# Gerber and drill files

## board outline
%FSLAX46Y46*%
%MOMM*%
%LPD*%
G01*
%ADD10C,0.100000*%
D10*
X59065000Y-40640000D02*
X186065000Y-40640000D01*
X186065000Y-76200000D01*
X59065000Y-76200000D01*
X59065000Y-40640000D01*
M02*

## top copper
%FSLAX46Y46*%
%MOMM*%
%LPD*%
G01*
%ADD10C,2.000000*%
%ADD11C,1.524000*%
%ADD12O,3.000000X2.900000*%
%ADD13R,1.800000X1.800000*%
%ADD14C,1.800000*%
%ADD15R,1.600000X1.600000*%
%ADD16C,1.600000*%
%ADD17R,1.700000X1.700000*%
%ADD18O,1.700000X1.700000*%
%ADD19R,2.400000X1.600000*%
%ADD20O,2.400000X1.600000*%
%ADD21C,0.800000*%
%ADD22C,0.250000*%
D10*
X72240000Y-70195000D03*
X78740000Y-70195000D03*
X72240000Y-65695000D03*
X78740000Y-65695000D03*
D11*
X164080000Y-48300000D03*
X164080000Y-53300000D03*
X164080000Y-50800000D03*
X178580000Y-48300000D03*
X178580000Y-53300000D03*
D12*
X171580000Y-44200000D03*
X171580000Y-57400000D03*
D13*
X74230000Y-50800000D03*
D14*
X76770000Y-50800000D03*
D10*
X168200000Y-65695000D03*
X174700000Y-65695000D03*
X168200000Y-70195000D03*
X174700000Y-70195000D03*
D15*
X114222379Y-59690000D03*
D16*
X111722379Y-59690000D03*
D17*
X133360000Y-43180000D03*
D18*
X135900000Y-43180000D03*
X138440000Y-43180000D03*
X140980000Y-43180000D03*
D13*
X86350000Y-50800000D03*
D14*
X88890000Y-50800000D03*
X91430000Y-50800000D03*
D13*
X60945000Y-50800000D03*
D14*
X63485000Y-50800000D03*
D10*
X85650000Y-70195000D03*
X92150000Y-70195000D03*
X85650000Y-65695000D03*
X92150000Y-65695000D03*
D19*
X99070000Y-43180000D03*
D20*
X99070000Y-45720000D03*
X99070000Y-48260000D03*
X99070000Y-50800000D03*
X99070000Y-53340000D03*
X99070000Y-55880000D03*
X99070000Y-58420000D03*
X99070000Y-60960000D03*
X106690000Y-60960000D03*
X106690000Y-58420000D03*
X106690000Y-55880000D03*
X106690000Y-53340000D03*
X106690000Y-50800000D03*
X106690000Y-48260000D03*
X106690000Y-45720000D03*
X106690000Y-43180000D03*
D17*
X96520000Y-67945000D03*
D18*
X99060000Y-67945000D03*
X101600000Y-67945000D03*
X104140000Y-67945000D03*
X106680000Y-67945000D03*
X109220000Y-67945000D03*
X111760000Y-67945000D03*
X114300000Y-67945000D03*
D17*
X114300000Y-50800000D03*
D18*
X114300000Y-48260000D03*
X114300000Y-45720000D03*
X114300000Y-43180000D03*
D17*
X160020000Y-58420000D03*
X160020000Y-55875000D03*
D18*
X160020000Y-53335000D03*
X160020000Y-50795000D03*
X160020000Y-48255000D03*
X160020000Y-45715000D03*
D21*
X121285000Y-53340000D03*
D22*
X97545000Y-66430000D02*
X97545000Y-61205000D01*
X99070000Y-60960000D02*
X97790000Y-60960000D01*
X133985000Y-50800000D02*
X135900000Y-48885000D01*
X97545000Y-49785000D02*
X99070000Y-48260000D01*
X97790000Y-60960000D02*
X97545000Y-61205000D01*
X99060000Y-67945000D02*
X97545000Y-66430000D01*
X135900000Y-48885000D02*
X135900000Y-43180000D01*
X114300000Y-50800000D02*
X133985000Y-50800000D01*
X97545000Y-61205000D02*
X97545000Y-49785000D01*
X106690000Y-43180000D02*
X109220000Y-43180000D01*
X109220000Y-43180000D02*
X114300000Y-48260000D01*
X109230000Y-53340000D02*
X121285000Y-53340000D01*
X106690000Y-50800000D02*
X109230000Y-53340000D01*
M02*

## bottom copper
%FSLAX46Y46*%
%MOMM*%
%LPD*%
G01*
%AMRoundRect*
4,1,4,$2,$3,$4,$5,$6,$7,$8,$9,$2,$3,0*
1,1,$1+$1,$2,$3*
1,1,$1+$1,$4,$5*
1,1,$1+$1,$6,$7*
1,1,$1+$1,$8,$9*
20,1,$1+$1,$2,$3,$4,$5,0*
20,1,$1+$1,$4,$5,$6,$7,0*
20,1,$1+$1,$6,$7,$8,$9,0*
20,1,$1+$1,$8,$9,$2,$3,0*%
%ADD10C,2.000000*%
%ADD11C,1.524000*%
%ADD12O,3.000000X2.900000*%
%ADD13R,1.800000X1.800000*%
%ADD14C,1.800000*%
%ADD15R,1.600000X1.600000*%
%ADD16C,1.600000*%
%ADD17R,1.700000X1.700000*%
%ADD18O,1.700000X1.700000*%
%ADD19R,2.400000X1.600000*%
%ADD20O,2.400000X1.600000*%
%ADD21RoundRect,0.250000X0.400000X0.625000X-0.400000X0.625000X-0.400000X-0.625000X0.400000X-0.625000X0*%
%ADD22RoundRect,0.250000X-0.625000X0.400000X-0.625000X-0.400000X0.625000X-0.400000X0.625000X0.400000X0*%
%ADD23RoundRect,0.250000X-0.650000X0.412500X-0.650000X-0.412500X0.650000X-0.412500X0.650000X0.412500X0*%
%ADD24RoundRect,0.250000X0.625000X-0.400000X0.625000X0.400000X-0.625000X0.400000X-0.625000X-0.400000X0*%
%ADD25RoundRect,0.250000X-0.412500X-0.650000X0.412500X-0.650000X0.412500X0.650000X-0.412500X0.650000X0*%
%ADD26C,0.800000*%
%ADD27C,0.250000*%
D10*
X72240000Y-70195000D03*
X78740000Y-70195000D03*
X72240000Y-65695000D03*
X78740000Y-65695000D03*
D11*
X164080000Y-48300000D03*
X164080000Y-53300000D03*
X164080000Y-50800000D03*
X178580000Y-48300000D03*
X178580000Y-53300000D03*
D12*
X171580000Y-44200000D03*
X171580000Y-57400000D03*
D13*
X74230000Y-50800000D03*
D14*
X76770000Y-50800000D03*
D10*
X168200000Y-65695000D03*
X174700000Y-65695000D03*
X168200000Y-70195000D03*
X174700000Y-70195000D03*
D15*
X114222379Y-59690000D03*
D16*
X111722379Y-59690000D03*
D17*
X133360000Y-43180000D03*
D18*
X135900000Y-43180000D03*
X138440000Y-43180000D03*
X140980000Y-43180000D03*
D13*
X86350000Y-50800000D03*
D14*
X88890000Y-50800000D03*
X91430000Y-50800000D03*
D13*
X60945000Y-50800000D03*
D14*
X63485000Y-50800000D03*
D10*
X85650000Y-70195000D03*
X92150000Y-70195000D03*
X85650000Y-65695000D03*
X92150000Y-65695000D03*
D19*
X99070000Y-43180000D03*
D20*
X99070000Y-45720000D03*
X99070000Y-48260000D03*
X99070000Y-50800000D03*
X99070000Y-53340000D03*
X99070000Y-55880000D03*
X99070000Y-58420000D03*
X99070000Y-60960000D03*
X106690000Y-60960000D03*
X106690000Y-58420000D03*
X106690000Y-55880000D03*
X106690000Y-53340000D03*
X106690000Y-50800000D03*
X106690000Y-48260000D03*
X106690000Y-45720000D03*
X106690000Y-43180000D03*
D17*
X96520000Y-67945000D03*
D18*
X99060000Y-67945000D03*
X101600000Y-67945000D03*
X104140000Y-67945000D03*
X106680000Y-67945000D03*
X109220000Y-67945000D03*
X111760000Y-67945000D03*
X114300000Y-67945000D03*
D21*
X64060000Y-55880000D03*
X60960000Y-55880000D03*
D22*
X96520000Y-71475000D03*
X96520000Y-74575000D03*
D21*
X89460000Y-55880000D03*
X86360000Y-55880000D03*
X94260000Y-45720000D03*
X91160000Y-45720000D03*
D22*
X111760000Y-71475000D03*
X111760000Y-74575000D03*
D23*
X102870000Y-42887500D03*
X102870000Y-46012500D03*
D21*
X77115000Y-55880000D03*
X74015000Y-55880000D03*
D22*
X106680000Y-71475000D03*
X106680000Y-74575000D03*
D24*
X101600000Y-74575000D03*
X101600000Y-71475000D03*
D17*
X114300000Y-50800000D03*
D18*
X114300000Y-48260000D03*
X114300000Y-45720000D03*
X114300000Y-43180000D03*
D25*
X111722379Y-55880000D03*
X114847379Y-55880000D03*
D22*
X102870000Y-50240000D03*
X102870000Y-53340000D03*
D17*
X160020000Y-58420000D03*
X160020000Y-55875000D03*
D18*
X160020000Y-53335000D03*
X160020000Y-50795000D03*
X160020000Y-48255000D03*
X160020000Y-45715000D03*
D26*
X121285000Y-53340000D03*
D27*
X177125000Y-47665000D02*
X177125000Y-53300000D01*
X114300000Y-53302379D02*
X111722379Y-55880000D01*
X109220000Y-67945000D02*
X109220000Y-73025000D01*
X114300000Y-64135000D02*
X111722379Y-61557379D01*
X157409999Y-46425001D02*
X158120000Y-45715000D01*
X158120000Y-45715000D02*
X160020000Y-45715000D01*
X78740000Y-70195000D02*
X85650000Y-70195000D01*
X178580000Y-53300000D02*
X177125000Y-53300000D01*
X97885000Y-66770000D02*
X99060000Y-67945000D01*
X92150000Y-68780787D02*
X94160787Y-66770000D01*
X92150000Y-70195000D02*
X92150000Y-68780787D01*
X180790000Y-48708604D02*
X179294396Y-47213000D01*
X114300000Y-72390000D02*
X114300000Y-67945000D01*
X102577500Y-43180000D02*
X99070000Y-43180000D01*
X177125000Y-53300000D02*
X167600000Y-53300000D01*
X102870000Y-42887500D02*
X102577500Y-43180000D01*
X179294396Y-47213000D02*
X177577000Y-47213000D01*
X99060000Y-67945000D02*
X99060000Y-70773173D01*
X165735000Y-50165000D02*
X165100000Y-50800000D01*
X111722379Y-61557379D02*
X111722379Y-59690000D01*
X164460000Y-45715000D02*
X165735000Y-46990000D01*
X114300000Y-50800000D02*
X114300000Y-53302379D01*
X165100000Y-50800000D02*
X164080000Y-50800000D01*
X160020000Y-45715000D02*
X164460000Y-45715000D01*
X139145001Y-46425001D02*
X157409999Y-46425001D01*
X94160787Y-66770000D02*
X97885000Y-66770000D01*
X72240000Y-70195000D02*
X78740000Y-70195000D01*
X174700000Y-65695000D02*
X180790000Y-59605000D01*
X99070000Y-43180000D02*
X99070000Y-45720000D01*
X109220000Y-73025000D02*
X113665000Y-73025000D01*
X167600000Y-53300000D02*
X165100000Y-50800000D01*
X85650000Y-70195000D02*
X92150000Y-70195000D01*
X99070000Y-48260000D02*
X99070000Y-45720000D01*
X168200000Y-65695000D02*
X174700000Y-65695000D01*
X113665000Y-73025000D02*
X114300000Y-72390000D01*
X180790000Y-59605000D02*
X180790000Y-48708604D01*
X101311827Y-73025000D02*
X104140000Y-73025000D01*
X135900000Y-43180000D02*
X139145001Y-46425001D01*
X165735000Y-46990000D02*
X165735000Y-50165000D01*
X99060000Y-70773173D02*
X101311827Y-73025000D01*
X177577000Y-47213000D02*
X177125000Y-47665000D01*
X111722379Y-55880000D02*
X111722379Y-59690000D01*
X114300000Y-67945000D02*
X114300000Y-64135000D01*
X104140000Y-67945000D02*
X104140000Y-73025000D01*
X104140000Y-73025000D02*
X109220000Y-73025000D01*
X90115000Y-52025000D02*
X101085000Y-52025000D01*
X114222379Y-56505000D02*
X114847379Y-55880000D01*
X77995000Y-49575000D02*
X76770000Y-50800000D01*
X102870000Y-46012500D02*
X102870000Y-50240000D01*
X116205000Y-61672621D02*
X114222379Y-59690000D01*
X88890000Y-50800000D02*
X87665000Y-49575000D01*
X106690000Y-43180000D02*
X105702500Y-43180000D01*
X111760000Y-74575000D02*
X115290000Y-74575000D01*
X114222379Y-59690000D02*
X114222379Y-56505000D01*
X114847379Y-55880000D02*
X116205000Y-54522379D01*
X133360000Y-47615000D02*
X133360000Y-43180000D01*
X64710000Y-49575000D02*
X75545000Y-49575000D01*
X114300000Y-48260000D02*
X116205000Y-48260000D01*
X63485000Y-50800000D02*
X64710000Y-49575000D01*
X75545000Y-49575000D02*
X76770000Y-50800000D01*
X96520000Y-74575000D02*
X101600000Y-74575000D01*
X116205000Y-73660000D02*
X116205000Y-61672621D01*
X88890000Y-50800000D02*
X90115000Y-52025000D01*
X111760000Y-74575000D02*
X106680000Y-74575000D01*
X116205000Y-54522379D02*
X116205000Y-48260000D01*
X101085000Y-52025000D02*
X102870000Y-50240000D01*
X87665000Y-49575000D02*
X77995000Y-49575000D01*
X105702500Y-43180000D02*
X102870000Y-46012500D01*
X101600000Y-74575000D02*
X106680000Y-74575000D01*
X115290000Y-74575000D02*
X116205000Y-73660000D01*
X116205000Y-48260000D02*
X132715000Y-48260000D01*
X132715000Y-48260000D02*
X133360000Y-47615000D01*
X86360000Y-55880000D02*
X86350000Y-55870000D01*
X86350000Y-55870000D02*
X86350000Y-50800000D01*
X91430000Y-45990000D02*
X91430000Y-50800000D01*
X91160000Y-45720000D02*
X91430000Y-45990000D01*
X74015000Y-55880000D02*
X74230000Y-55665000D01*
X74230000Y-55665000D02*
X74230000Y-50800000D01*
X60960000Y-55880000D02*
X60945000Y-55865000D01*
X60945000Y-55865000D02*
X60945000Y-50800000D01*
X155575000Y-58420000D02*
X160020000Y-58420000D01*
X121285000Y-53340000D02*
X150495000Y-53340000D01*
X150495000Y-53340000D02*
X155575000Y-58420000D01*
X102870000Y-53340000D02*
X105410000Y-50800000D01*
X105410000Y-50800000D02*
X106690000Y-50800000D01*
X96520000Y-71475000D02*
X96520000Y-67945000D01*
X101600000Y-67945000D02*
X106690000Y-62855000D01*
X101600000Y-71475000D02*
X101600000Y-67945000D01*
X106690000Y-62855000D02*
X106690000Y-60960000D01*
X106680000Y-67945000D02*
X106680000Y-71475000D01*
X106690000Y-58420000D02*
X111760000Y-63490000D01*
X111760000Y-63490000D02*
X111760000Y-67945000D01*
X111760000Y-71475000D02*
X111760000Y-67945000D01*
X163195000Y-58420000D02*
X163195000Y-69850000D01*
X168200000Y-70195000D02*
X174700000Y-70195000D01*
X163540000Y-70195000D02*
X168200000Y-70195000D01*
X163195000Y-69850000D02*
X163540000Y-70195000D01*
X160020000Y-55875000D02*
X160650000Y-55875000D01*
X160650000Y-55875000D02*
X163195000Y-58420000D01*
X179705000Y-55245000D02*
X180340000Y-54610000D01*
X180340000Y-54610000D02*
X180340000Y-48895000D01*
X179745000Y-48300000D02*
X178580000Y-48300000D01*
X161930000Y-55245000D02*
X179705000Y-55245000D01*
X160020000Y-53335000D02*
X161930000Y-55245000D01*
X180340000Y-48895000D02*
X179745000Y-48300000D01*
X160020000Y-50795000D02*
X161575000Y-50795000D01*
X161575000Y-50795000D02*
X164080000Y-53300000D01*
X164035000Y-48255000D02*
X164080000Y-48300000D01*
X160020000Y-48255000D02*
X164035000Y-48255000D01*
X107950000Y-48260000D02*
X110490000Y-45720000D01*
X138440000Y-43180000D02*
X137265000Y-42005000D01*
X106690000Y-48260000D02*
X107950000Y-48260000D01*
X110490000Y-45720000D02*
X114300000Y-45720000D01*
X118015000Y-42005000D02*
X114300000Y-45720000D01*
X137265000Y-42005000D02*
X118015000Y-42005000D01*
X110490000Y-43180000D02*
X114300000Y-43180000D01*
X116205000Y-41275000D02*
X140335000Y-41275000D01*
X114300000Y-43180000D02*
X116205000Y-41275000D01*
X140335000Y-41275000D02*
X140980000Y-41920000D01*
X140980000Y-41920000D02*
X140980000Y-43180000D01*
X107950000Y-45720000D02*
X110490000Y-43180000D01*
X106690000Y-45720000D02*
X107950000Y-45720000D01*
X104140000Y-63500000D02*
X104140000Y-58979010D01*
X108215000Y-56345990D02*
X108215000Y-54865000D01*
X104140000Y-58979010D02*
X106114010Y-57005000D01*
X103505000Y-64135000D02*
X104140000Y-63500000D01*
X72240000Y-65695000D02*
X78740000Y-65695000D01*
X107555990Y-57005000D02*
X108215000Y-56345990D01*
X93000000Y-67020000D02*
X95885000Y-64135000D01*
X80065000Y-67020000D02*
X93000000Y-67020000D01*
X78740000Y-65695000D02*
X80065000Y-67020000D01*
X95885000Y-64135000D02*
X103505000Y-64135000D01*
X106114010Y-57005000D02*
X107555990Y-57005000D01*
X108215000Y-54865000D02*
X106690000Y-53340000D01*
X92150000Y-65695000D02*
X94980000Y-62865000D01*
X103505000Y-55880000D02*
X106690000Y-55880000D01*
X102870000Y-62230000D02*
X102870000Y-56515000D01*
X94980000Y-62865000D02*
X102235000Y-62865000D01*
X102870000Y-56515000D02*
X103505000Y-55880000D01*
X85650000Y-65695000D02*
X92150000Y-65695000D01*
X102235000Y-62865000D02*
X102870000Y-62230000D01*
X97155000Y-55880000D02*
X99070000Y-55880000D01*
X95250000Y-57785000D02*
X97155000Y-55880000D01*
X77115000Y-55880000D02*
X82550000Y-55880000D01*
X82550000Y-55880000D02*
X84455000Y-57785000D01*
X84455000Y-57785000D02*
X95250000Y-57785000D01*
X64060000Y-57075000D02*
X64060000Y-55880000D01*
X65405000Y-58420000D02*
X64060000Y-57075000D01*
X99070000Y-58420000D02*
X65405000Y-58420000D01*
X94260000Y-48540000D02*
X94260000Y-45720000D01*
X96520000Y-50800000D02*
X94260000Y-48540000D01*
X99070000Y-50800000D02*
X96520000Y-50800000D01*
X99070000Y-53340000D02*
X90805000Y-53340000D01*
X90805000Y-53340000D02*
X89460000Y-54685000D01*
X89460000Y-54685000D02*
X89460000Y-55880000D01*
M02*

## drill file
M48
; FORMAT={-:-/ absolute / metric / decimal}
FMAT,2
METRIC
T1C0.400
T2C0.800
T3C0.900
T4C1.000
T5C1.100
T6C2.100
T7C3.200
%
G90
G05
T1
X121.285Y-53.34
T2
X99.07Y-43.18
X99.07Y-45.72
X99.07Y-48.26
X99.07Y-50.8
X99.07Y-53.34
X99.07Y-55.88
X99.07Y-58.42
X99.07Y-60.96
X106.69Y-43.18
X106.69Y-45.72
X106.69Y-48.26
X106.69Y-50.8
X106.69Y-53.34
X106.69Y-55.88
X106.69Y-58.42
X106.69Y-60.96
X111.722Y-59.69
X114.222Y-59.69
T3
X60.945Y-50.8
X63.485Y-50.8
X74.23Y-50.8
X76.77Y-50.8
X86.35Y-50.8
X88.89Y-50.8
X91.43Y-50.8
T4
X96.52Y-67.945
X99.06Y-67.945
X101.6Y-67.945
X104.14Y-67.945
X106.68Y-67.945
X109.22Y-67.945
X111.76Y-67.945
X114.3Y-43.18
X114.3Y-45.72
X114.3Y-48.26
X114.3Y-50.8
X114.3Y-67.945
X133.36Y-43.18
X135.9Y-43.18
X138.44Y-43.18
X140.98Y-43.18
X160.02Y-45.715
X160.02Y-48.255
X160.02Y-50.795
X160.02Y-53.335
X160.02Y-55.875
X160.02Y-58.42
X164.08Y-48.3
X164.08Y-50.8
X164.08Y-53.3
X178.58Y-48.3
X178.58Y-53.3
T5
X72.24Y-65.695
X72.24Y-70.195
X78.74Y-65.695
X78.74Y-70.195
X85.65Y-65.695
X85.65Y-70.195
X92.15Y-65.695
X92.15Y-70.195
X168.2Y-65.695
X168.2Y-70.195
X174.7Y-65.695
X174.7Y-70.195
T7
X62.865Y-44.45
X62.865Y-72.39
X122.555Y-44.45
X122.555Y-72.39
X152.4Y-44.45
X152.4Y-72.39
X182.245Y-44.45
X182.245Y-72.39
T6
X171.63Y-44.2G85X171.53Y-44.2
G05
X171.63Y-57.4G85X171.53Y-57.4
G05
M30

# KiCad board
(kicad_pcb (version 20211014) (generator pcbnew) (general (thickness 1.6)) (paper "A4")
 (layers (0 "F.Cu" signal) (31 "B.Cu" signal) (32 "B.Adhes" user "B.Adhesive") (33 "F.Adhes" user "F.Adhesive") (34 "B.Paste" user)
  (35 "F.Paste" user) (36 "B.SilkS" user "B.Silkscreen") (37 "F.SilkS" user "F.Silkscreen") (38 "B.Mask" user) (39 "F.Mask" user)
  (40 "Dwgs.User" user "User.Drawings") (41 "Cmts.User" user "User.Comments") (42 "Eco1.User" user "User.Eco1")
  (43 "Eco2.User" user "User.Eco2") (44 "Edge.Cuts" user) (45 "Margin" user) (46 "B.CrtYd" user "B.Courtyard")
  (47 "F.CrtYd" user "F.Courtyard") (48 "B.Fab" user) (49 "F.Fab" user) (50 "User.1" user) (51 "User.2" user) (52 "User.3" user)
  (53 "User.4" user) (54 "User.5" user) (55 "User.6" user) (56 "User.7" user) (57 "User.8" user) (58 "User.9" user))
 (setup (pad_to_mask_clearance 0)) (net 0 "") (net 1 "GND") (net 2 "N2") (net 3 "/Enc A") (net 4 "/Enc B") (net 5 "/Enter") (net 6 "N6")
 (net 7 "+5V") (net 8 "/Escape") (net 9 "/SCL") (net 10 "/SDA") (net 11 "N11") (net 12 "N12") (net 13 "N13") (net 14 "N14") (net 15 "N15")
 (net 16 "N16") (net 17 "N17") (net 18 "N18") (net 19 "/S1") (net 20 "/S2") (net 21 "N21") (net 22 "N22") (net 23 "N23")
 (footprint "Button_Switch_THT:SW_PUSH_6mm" (layer "F.Cu") (at 78.74 70.195 180)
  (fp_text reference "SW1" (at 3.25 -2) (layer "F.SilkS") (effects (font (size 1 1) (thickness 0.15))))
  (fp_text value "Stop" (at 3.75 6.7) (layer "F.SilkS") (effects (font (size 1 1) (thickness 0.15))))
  (pad "1" thru_hole circle (at 6.5 0 270) (size 2 2) (drill 1.1) (layers *.Cu *.Mask) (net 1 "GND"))
  (pad "1" thru_hole circle (at 0 0 270) (size 2 2) (drill 1.1) (layers *.Cu *.Mask) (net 1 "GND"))
  (pad "2" thru_hole circle (at 6.5 4.5 270) (size 2 2) (drill 1.1) (layers *.Cu *.Mask) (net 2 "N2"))
  (pad "2" thru_hole circle (at 0 4.5 270) (size 2 2) (drill 1.1) (layers *.Cu *.Mask) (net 2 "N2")))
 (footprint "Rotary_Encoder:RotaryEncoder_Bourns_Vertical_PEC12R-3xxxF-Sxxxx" (layer "F.Cu") (at 164.08 48.3)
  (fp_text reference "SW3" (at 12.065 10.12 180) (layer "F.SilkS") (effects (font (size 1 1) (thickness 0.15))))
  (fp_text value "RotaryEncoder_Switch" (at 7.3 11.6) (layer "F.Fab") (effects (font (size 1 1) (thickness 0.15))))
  (pad "A" thru_hole circle (at 0 0 270) (size 1.524 1.524) (drill 1) (layers *.Cu *.Mask) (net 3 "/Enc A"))
  (pad "B" thru_hole circle (at 0 5 270) (size 1.524 1.524) (drill 1) (layers *.Cu *.Mask) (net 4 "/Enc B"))
  (pad "C" thru_hole circle (at 0 2.5 270) (size 1.524 1.524) (drill 1) (layers *.Cu *.Mask) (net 1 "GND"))
  (pad "S1" thru_hole circle (at 14.5 0 270) (size 1.524 1.524) (drill 1) (layers *.Cu *.Mask) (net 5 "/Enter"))
  (pad "S2" thru_hole circle (at 14.5 5 270) (size 1.524 1.524) (drill 1) (layers *.Cu *.Mask) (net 1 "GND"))
  (pad "SH" thru_hole oval (at 7.5 -4.1 270) (size 2.9 3) (drill oval 2.1 2.2) (layers *.Cu *.Mask))
  (pad "SH" thru_hole oval (at 7.5 9.1 270) (size 2.9 3) (drill oval 2.1 2.2) (layers *.Cu *.Mask)))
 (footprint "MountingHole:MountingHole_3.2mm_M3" (layer "F.Cu") (at 62.865 72.39)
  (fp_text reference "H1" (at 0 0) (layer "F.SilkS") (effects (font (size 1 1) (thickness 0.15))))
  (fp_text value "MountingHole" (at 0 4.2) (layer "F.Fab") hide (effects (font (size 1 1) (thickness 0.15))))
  (pad "" np_thru_hole circle (at 0 0) (size 3.2 3.2) (drill 3.2) (layers *.Cu *.Mask)))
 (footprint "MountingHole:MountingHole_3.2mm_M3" (layer "F.Cu") (at 122.555 44.45)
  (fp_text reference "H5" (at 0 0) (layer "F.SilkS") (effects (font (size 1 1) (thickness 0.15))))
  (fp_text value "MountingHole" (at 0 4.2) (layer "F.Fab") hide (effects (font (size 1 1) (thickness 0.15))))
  (pad "" np_thru_hole circle (at 0 0) (size 3.2 3.2) (drill 3.2) (layers *.Cu *.Mask)))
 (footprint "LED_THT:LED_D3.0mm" (layer "F.Cu") (at 74.23 50.8)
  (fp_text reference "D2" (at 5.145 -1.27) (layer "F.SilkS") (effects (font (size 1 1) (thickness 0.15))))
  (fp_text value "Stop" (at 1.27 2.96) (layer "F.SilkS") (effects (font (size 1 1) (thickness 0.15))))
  (pad "1" thru_hole rect (at 0 0) (size 1.8 1.8) (drill 0.9) (layers *.Cu *.Mask) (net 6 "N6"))
  (pad "2" thru_hole circle (at 2.54 0) (size 1.8 1.8) (drill 0.9) (layers *.Cu *.Mask) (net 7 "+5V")))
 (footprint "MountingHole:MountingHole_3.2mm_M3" (layer "F.Cu") (at 182.245 72.39)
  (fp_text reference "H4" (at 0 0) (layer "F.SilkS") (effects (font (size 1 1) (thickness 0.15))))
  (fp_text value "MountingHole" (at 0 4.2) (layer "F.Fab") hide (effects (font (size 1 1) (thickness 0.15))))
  (pad "" np_thru_hole circle (at 0 0) (size 3.2 3.2) (drill 3.2) (layers *.Cu *.Mask)))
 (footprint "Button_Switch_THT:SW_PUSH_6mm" (layer "F.Cu") (at 168.2 65.695)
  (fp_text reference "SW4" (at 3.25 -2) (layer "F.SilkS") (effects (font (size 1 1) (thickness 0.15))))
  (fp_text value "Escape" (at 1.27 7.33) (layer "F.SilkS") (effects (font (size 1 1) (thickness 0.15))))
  (pad "1" thru_hole circle (at 0 0 90) (size 2 2) (drill 1.1) (layers *.Cu *.Mask) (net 1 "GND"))
  (pad "1" thru_hole circle (at 6.5 0 90) (size 2 2) (drill 1.1) (layers *.Cu *.Mask) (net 1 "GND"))
  (pad "2" thru_hole circle (at 0 4.5 90) (size 2 2) (drill 1.1) (layers *.Cu *.Mask) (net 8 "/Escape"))
  (pad "2" thru_hole circle (at 6.5 4.5 90) (size 2 2) (drill 1.1) (layers *.Cu *.Mask) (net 8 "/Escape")))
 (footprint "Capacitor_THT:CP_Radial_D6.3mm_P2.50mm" (layer "F.Cu") (at 114.222379 59.69 180)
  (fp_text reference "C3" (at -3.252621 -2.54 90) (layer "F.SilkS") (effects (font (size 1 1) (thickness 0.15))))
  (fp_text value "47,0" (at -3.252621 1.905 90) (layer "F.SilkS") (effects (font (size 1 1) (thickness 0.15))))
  (pad "1" thru_hole rect (at 0 0 180) (size 1.6 1.6) (drill 0.8) (layers *.Cu *.Mask) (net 7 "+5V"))
  (pad "2" thru_hole circle (at 2.5 0 180) (size 1.6 1.6) (drill 0.8) (layers *.Cu *.Mask) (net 1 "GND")))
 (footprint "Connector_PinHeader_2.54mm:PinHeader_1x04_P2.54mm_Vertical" (layer "F.Cu") (at 133.36 43.18 90)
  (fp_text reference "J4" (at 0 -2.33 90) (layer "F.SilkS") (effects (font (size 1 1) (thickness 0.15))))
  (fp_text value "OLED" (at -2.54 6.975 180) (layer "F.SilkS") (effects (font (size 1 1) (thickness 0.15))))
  (pad "1" thru_hole rect (at 0 0 90) (size 1.7 1.7) (drill 1) (layers *.Cu *.Mask) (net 7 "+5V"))
  (pad "2" thru_hole oval (at 0 2.54 90) (size 1.7 1.7) (drill 1) (layers *.Cu *.Mask) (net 1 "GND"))
  (pad "3" thru_hole oval (at 0 5.08 90) (size 1.7 1.7) (drill 1) (layers *.Cu *.Mask) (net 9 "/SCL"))
  (pad "4" thru_hole oval (at 0 7.62 90) (size 1.7 1.7) (drill 1) (layers *.Cu *.Mask) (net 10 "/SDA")))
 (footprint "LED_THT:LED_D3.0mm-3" (layer "F.Cu") (at 86.35 50.8)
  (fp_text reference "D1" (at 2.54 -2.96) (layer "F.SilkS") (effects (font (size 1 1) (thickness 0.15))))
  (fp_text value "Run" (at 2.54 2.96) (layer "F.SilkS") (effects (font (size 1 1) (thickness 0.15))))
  (pad "1" thru_hole rect (at 0 0) (size 1.8 1.8) (drill 0.9) (layers *.Cu *.Mask) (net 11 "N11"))
  (pad "2" thru_hole circle (at 2.54 0) (size 1.8 1.8) (drill 0.9) (layers *.Cu *.Mask) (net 7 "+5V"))
  (pad "3" thru_hole circle (at 5.08 0) (size 1.8 1.8) (drill 0.9) (layers *.Cu *.Mask) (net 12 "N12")))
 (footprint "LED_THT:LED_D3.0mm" (layer "F.Cu") (at 60.945 50.8)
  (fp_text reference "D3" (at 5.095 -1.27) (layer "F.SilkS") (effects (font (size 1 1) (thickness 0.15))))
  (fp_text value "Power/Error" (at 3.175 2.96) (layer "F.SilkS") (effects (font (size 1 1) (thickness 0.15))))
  (pad "1" thru_hole rect (at 0 0) (size 1.8 1.8) (drill 0.9) (layers *.Cu *.Mask) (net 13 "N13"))
  (pad "2" thru_hole circle (at 2.54 0) (size 1.8 1.8) (drill 0.9) (layers *.Cu *.Mask) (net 7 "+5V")))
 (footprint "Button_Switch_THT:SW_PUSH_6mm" (layer "F.Cu") (at 92.15 70.195 180)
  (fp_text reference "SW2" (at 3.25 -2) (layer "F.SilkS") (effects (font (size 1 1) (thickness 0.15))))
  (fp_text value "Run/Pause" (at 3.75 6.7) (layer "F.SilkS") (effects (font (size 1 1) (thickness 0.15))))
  (pad "1" thru_hole circle (at 6.5 0 270) (size 2 2) (drill 1.1) (layers *.Cu *.Mask) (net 1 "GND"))
  (pad "1" thru_hole circle (at 0 0 270) (size 2 2) (drill 1.1) (layers *.Cu *.Mask) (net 1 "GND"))
  (pad "2" thru_hole circle (at 6.5 4.5 270) (size 2 2) (drill 1.1) (layers *.Cu *.Mask) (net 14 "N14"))
  (pad "2" thru_hole circle (at 0 4.5 270) (size 2 2) (drill 1.1) (layers *.Cu *.Mask) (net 14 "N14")))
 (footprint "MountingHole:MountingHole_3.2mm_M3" (layer "F.Cu") (at 182.245 44.45)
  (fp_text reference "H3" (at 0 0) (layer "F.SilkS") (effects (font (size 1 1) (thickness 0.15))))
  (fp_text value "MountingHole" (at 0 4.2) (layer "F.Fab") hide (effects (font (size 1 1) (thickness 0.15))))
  (pad "" np_thru_hole circle (at 0 0) (size 3.2 3.2) (drill 3.2) (layers *.Cu *.Mask)))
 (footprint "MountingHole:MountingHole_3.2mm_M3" (layer "F.Cu") (at 62.865 44.45)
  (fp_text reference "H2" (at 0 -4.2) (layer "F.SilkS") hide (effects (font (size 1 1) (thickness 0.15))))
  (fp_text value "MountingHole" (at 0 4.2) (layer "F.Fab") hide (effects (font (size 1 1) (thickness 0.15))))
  (pad "" np_thru_hole circle (at 0 0) (size 3.2 3.2) (drill 3.2) (layers *.Cu *.Mask)))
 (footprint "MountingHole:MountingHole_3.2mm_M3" (layer "F.Cu") (at 152.4 72.39)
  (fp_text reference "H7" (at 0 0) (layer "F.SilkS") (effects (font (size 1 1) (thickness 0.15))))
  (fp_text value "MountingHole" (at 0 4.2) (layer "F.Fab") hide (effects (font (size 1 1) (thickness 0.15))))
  (pad "" np_thru_hole circle (at 0 0) (size 3.2 3.2) (drill 3.2) (layers *.Cu *.Mask)))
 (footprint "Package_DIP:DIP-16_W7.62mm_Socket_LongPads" (layer "F.Cu") (at 99.07 43.18)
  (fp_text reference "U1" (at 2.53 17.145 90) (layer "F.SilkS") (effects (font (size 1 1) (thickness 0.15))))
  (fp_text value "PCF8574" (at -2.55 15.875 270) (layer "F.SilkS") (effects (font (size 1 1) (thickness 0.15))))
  (pad "1" thru_hole rect (at 0 0) (size 2.4 1.6) (drill 0.8) (layers *.Cu *.Mask) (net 1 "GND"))
  (pad "2" thru_hole oval (at 0 2.54) (size 2.4 1.6) (drill 0.8) (layers *.Cu *.Mask) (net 1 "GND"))
  (pad "3" thru_hole oval (at 0 5.08) (size 2.4 1.6) (drill 0.8) (layers *.Cu *.Mask) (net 1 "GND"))
  (pad "4" thru_hole oval (at 0 7.62) (size 2.4 1.6) (drill 0.8) (layers *.Cu *.Mask) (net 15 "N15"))
  (pad "5" thru_hole oval (at 0 10.16) (size 2.4 1.6) (drill 0.8) (layers *.Cu *.Mask) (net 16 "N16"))
  (pad "6" thru_hole oval (at 0 12.7) (size 2.4 1.6) (drill 0.8) (layers *.Cu *.Mask) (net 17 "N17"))
  (pad "7" thru_hole oval (at 0 15.24) (size 2.4 1.6) (drill 0.8) (layers *.Cu *.Mask) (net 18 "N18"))
  (pad "8" thru_hole oval (at 0 17.78) (size 2.4 1.6) (drill 0.8) (layers *.Cu *.Mask) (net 1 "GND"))
  (pad "9" thru_hole oval (at 7.62 17.78) (size 2.4 1.6) (drill 0.8) (layers *.Cu *.Mask) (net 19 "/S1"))
  (pad "10" thru_hole oval (at 7.62 15.24) (size 2.4 1.6) (drill 0.8) (layers *.Cu *.Mask) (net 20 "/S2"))
  (pad "11" thru_hole oval (at 7.62 12.7) (size 2.4 1.6) (drill 0.8) (layers *.Cu *.Mask) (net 14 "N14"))
  (pad "12" thru_hole oval (at 7.62 10.16) (size 2.4 1.6) (drill 0.8) (layers *.Cu *.Mask) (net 2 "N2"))
  (pad "13" thru_hole oval (at 7.62 7.62) (size 2.4 1.6) (drill 0.8) (layers *.Cu *.Mask) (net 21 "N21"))
  (pad "14" thru_hole oval (at 7.62 5.08) (size 2.4 1.6) (drill 0.8) (layers *.Cu *.Mask) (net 9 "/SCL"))
  (pad "15" thru_hole oval (at 7.62 2.54) (size 2.4 1.6) (drill 0.8) (layers *.Cu *.Mask) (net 10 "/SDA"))
  (pad "16" thru_hole oval (at 7.62 0) (size 2.4 1.6) (drill 0.8) (layers *.Cu *.Mask) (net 7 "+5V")))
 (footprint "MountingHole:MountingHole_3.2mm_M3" (layer "F.Cu") (at 152.4 44.45)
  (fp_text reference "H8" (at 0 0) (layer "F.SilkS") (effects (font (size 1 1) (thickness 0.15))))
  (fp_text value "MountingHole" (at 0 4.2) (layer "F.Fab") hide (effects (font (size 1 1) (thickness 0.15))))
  (pad "" np_thru_hole circle (at 0 0) (size 3.2 3.2) (drill 3.2) (layers *.Cu *.Mask)))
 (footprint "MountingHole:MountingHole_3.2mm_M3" (layer "F.Cu") (at 122.555 72.39)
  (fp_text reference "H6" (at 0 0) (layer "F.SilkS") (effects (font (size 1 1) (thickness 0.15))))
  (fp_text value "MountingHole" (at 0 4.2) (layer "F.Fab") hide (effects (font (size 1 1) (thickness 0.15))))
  (pad "" np_thru_hole circle (at 0 0) (size 3.2 3.2) (drill 3.2) (layers *.Cu *.Mask)))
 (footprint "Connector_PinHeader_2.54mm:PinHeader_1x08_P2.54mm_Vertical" (layer "B.Cu") (at 96.52 67.945 -90)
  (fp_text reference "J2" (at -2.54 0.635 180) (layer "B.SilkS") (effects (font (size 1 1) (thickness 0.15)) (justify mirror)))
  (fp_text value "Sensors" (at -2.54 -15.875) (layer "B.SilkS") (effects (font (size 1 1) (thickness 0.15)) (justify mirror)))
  (pad "1" thru_hole rect (at 0 0 270) (size 1.7 1.7) (drill 1) (layers *.Cu *.Mask) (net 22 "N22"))
  (pad "2" thru_hole oval (at 0 -2.54 270) (size 1.7 1.7) (drill 1) (layers *.Cu *.Mask) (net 1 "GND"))
  (pad "3" thru_hole oval (at 0 -5.08 270) (size 1.7 1.7) (drill 1) (layers *.Cu *.Mask) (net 19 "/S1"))
  (pad "4" thru_hole oval (at 0 -7.62 270) (size 1.7 1.7) (drill 1) (layers *.Cu *.Mask) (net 1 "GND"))
  (pad "5" thru_hole oval (at 0 -10.16 270) (size 1.7 1.7) (drill 1) (layers *.Cu *.Mask) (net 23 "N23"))
  (pad "6" thru_hole oval (at 0 -12.7 270) (size 1.7 1.7) (drill 1) (layers *.Cu *.Mask) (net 1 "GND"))
  (pad "7" thru_hole oval (at 0 -15.24 270) (size 1.7 1.7) (drill 1) (layers *.Cu *.Mask) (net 20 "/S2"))
  (pad "8" thru_hole oval (at 0 -17.78 270) (size 1.7 1.7) (drill 1) (layers *.Cu *.Mask) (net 1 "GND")))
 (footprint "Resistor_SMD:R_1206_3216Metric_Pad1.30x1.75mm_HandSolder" (layer "B.Cu") (at 62.51 55.88 180)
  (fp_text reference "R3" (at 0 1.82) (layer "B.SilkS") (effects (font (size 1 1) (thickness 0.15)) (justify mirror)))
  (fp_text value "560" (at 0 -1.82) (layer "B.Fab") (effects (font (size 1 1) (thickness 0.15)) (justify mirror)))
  (pad "1" smd roundrect (at -1.55 0 180) (size 1.3 1.75) (layers "B.Cu" "B.Paste" "B.Mask") (roundrect_rratio 0.192308) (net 18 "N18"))
  (pad "2" smd roundrect (at 1.55 0 180) (size 1.3 1.75) (layers "B.Cu" "B.Paste" "B.Mask") (roundrect_rratio 0.192308) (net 13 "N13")))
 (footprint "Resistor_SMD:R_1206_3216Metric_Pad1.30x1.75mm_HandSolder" (layer "B.Cu") (at 96.52 73.025 -90)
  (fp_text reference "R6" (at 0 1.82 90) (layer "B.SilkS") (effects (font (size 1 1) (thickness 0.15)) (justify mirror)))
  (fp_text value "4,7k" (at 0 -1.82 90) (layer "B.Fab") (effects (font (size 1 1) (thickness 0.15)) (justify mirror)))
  (pad "1" smd roundrect (at -1.55 0 270) (size 1.3 1.75) (layers "B.Cu" "B.Paste" "B.Mask") (roundrect_rratio 0.192308) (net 22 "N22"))
  (pad "2" smd roundrect (at 1.55 0 270) (size 1.3 1.75) (layers "B.Cu" "B.Paste" "B.Mask") (roundrect_rratio 0.192308) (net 7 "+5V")))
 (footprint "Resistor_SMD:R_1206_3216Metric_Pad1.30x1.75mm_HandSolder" (layer "B.Cu") (at 87.91 55.88 180)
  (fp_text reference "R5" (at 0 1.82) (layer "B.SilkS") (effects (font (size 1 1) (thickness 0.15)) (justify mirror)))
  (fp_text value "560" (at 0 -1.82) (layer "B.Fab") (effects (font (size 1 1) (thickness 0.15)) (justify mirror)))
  (pad "1" smd roundrect (at -1.55 0 180) (size 1.3 1.75) (layers "B.Cu" "B.Paste" "B.Mask") (roundrect_rratio 0.192308) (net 16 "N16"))
  (pad "2" smd roundrect (at 1.55 0 180) (size 1.3 1.75) (layers "B.Cu" "B.Paste" "B.Mask") (roundrect_rratio 0.192308) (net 11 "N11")))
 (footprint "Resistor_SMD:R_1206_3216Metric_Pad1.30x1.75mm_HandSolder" (layer "B.Cu") (at 92.71 45.72 180)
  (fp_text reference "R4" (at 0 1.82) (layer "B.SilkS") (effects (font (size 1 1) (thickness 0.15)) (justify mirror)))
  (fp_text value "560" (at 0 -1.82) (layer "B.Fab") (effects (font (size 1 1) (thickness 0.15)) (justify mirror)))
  (pad "1" smd roundrect (at -1.55 0 180) (size 1.3 1.75) (layers "B.Cu" "B.Paste" "B.Mask") (roundrect_rratio 0.192308) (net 15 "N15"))
  (pad "2" smd roundrect (at 1.55 0 180) (size 1.3 1.75) (layers "B.Cu" "B.Paste" "B.Mask") (roundrect_rratio 0.192308) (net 12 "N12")))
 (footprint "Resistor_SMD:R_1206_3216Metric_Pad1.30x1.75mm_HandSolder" (layer "B.Cu") (at 111.76 73.025 -90)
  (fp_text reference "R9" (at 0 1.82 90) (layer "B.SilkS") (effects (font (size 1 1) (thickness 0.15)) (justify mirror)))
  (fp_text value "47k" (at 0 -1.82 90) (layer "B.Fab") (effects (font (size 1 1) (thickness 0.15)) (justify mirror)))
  (pad "1" smd roundrect (at -1.55 0 270) (size 1.3 1.75) (layers "B.Cu" "B.Paste" "B.Mask") (roundrect_rratio 0.192308) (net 20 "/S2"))
  (pad "2" smd roundrect (at 1.55 0 270) (size 1.3 1.75) (layers "B.Cu" "B.Paste" "B.Mask") (roundrect_rratio 0.192308) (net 7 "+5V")))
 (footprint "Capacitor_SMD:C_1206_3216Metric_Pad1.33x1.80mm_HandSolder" (layer "B.Cu") (at 102.87 44.45 -90)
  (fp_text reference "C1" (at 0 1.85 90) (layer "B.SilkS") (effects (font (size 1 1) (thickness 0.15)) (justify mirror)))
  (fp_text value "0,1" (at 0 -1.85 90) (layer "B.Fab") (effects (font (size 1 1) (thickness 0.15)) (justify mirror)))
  (pad "1" smd roundrect (at -1.5625 0 270) (size 1.325 1.8) (layers "B.Cu" "B.Paste" "B.Mask") (roundrect_rratio 0.188679) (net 1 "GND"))
  (pad "2" smd roundrect (at 1.5625 0 270) (size 1.325 1.8) (layers "B.Cu" "B.Paste" "B.Mask") (roundrect_rratio 0.188679) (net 7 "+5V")))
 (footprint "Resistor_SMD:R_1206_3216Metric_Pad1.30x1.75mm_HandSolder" (layer "B.Cu") (at 75.565 55.88 180)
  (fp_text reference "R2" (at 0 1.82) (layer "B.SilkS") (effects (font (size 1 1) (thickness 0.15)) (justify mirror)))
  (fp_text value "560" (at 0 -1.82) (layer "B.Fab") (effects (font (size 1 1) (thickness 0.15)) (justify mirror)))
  (pad "1" smd roundrect (at -1.55 0 180) (size 1.3 1.75) (layers "B.Cu" "B.Paste" "B.Mask") (roundrect_rratio 0.192308) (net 17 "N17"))
  (pad "2" smd roundrect (at 1.55 0 180) (size 1.3 1.75) (layers "B.Cu" "B.Paste" "B.Mask") (roundrect_rratio 0.192308) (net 6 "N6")))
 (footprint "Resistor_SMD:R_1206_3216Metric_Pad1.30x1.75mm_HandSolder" (layer "B.Cu") (at 106.68 73.025 -90)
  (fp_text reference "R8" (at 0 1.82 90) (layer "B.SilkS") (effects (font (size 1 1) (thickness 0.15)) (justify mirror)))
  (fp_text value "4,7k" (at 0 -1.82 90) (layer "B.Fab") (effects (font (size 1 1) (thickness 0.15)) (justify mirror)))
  (pad "1" smd roundrect (at -1.55 0 270) (size 1.3 1.75) (layers "B.Cu" "B.Paste" "B.Mask") (roundrect_rratio 0.192308) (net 23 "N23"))
  (pad "2" smd roundrect (at 1.55 0 270) (size 1.3 1.75) (layers "B.Cu" "B.Paste" "B.Mask") (roundrect_rratio 0.192308) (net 7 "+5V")))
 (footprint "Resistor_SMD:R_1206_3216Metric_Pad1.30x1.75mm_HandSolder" (layer "B.Cu") (at 101.6 73.025 90)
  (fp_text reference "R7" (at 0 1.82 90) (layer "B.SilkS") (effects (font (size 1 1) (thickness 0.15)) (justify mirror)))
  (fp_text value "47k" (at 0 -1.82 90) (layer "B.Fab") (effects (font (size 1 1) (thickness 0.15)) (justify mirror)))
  (pad "1" smd roundrect (at -1.55 0 90) (size 1.3 1.75) (layers "B.Cu" "B.Paste" "B.Mask") (roundrect_rratio 0.192308) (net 7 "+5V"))
  (pad "2" smd roundrect (at 1.55 0 90) (size 1.3 1.75) (layers "B.Cu" "B.Paste" "B.Mask") (roundrect_rratio 0.192308) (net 19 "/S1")))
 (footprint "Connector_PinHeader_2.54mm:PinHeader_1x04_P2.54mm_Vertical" (layer "B.Cu") (at 114.3 50.8)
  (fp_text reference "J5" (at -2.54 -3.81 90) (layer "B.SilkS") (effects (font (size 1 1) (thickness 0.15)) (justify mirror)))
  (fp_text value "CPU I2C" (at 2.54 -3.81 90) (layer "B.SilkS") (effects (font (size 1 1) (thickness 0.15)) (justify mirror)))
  (pad "1" thru_hole rect (at 0 0) (size 1.7 1.7) (drill 1) (layers *.Cu *.Mask) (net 1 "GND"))
  (pad "2" thru_hole oval (at 0 -2.54) (size 1.7 1.7) (drill 1) (layers *.Cu *.Mask) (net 7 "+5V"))
  (pad "3" thru_hole oval (at 0 -5.08) (size 1.7 1.7) (drill 1) (layers *.Cu *.Mask) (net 9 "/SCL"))
  (pad "4" thru_hole oval (at 0 -7.62) (size 1.7 1.7) (drill 1) (layers *.Cu *.Mask) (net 10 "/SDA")))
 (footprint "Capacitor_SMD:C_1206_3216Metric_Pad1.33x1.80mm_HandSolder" (layer "B.Cu") (at 113.284879 55.88)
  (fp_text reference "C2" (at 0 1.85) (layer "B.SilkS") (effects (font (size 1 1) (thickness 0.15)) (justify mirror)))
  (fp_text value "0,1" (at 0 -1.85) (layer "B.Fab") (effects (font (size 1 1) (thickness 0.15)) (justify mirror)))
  (pad "1" smd roundrect (at -1.5625 0) (size 1.325 1.8) (layers "B.Cu" "B.Paste" "B.Mask") (roundrect_rratio 0.188679) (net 1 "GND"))
  (pad "2" smd roundrect (at 1.5625 0) (size 1.325 1.8) (layers "B.Cu" "B.Paste" "B.Mask") (roundrect_rratio 0.188679) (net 7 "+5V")))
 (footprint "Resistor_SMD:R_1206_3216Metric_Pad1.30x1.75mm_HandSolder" (layer "B.Cu") (at 102.87 51.79 -90)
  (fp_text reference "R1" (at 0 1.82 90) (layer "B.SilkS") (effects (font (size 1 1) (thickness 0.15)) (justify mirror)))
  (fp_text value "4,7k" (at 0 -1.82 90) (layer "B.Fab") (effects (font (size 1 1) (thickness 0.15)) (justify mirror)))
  (pad "1" smd roundrect (at -1.55 0 270) (size 1.3 1.75) (layers "B.Cu" "B.Paste" "B.Mask") (roundrect_rratio 0.192308) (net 7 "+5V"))
  (pad "2" smd roundrect (at 1.55 0 270) (size 1.3 1.75) (layers "B.Cu" "B.Paste" "B.Mask") (roundrect_rratio 0.192308) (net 21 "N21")))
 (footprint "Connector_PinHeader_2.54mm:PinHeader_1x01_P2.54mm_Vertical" (layer "B.Cu") (at 160.02 58.42 180)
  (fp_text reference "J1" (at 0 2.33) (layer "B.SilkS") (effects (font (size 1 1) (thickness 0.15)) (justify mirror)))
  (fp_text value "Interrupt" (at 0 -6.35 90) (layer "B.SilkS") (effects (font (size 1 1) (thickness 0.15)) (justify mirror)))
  (pad "1" thru_hole rect (at 0 0 180) (size 1.7 1.7) (drill 1) (layers *.Cu *.Mask) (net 21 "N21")))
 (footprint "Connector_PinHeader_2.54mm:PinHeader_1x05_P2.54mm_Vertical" (layer "B.Cu") (at 160.02 55.875)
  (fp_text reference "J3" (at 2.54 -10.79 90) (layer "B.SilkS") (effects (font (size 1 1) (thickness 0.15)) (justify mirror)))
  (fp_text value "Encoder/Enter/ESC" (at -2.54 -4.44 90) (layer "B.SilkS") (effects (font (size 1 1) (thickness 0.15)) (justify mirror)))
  (pad "1" thru_hole rect (at 0 0) (size 1.7 1.7) (drill 1) (layers *.Cu *.Mask) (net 8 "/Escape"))
  (pad "2" thru_hole oval (at 0 -2.54) (size 1.7 1.7) (drill 1) (layers *.Cu *.Mask) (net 5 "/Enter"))
  (pad "3" thru_hole oval (at 0 -5.08) (size 1.7 1.7) (drill 1) (layers *.Cu *.Mask) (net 4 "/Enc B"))
  (pad "4" thru_hole oval (at 0 -7.62) (size 1.7 1.7) (drill 1) (layers *.Cu *.Mask) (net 3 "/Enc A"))
  (pad "5" thru_hole oval (at 0 -10.16) (size 1.7 1.7) (drill 1) (layers *.Cu *.Mask) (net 1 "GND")))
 (gr_rect (start 186.065 40.64) (end 59.065 76.2) (layer "Edge.Cuts") (width 0.1) (fill none))
 (segment (start 97.545 66.43) (end 97.545 61.205) (width 0.25) (layer "F.Cu") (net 1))
 (segment (start 99.07 60.96) (end 97.79 60.96) (width 0.25) (layer "F.Cu") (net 1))
 (segment (start 133.985 50.8) (end 135.9 48.885) (width 0.25) (layer "F.Cu") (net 1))
 (segment (start 97.545 49.785) (end 99.07 48.26) (width 0.25) (layer "F.Cu") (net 1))
 (segment (start 97.79 60.96) (end 97.545 61.205) (width 0.25) (layer "F.Cu") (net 1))
 (segment (start 99.06 67.945) (end 97.545 66.43) (width 0.25) (layer "F.Cu") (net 1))
 (segment (start 135.9 48.885) (end 135.9 43.18) (width 0.25) (layer "F.Cu") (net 1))
 (segment (start 114.3 50.8) (end 133.985 50.8) (width 0.25) (layer "F.Cu") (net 1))
 (segment (start 97.545 61.205) (end 97.545 49.785) (width 0.25) (layer "F.Cu") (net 1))
 (segment (start 177.125 47.665) (end 177.125 53.3) (width 0.25) (layer "B.Cu") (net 1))
 (segment (start 114.3 53.302379) (end 111.722379 55.88) (width 0.25) (layer "B.Cu") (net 1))
 (segment (start 109.22 67.945) (end 109.22 73.025) (width 0.25) (layer "B.Cu") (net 1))
 (segment (start 114.3 64.135) (end 111.722379 61.557379) (width 0.25) (layer "B.Cu") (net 1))
 (segment (start 157.409999 46.425001) (end 158.12 45.715) (width 0.25) (layer "B.Cu") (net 1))
 (segment (start 158.12 45.715) (end 160.02 45.715) (width 0.25) (layer "B.Cu") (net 1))
 (segment (start 78.74 70.195) (end 85.65 70.195) (width 0.25) (layer "B.Cu") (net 1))
 (segment (start 178.58 53.3) (end 177.125 53.3) (width 0.25) (layer "B.Cu") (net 1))
 (segment (start 97.885 66.77) (end 99.06 67.945) (width 0.25) (layer "B.Cu") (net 1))
 (segment (start 92.15 68.780787) (end 94.160787 66.77) (width 0.25) (layer "B.Cu") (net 1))
 (segment (start 92.15 70.195) (end 92.15 68.780787) (width 0.25) (layer "B.Cu") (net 1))
 (segment (start 180.79 48.708604) (end 179.294396 47.213) (width 0.25) (layer "B.Cu") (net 1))
 (segment (start 114.3 72.39) (end 114.3 67.945) (width 0.25) (layer "B.Cu") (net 1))
 (segment (start 102.5775 43.18) (end 99.07 43.18) (width 0.25) (layer "B.Cu") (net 1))
 (segment (start 177.125 53.3) (end 167.6 53.3) (width 0.25) (layer "B.Cu") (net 1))
 (segment (start 102.87 42.8875) (end 102.5775 43.18) (width 0.25) (layer "B.Cu") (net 1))
 (segment (start 179.294396 47.213) (end 177.577 47.213) (width 0.25) (layer "B.Cu") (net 1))
 (segment (start 99.06 67.945) (end 99.06 70.773173) (width 0.25) (layer "B.Cu") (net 1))
 (segment (start 165.735 50.165) (end 165.1 50.8) (width 0.25) (layer "B.Cu") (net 1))
 (segment (start 111.722379 61.557379) (end 111.722379 59.69) (width 0.25) (layer "B.Cu") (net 1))
 (segment (start 164.46 45.715) (end 165.735 46.99) (width 0.25) (layer "B.Cu") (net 1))
 (segment (start 114.3 50.8) (end 114.3 53.302379) (width 0.25) (layer "B.Cu") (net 1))
 (segment (start 165.1 50.8) (end 164.08 50.8) (width 0.25) (layer "B.Cu") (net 1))
 (segment (start 160.02 45.715) (end 164.46 45.715) (width 0.25) (layer "B.Cu") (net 1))
 (segment (start 139.145001 46.425001) (end 157.409999 46.425001) (width 0.25) (layer "B.Cu") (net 1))
 (segment (start 94.160787 66.77) (end 97.885 66.77) (width 0.25) (layer "B.Cu") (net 1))
 (segment (start 72.24 70.195) (end 78.74 70.195) (width 0.25) (layer "B.Cu") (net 1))
 (segment (start 174.7 65.695) (end 180.79 59.605) (width 0.25) (layer "B.Cu") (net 1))
 (segment (start 99.07 43.18) (end 99.07 45.72) (width 0.25) (layer "B.Cu") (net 1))
 (segment (start 109.22 73.025) (end 113.665 73.025) (width 0.25) (layer "B.Cu") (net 1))
 (segment (start 167.6 53.3) (end 165.1 50.8) (width 0.25) (layer "B.Cu") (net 1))
 (segment (start 85.65 70.195) (end 92.15 70.195) (width 0.25) (layer "B.Cu") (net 1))
 (segment (start 99.07 48.26) (end 99.07 45.72) (width 0.25) (layer "B.Cu") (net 1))
 (segment (start 168.2 65.695) (end 174.7 65.695) (width 0.25) (layer "B.Cu") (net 1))
 (segment (start 113.665 73.025) (end 114.3 72.39) (width 0.25) (layer "B.Cu") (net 1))
 (segment (start 180.79 59.605) (end 180.79 48.708604) (width 0.25) (layer "B.Cu") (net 1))
 (segment (start 101.311827 73.025) (end 104.14 73.025) (width 0.25) (layer "B.Cu") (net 1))
 (segment (start 135.9 43.18) (end 139.145001 46.425001) (width 0.25) (layer "B.Cu") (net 1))
 (segment (start 165.735 46.99) (end 165.735 50.165) (width 0.25) (layer "B.Cu") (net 1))
 (segment (start 99.06 70.773173) (end 101.311827 73.025) (width 0.25) (layer "B.Cu") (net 1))
 (segment (start 177.577 47.213) (end 177.125 47.665) (width 0.25) (layer "B.Cu") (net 1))
 (segment (start 111.722379 55.88) (end 111.722379 59.69) (width 0.25) (layer "B.Cu") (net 1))
 (segment (start 114.3 67.945) (end 114.3 64.135) (width 0.25) (layer "B.Cu") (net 1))
 (segment (start 104.14 67.945) (end 104.14 73.025) (width 0.25) (layer "B.Cu") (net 1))
 (segment (start 104.14 73.025) (end 109.22 73.025) (width 0.25) (layer "B.Cu") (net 1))
 (segment (start 106.69 43.18) (end 109.22 43.18) (width 0.25) (layer "F.Cu") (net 7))
 (segment (start 109.22 43.18) (end 114.3 48.26) (width 0.25) (layer "F.Cu") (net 7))
 (segment (start 90.115 52.025) (end 101.085 52.025) (width 0.25) (layer "B.Cu") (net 7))
 (segment (start 114.222379 56.505) (end 114.847379 55.88) (width 0.25) (layer "B.Cu") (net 7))
 (segment (start 77.995 49.575) (end 76.77 50.8) (width 0.25) (layer "B.Cu") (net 7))
 (segment (start 102.87 46.0125) (end 102.87 50.24) (width 0.25) (layer "B.Cu") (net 7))
 (segment (start 116.205 61.672621) (end 114.222379 59.69) (width 0.25) (layer "B.Cu") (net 7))
 (segment (start 88.89 50.8) (end 87.665 49.575) (width 0.25) (layer "B.Cu") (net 7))
 (segment (start 106.69 43.18) (end 105.7025 43.18) (width 0.25) (layer "B.Cu") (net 7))
 (segment (start 111.76 74.575) (end 115.29 74.575) (width 0.25) (layer "B.Cu") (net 7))
 (segment (start 114.222379 59.69) (end 114.222379 56.505) (width 0.25) (layer "B.Cu") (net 7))
 (segment (start 114.847379 55.88) (end 116.205 54.522379) (width 0.25) (layer "B.Cu") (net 7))
 (segment (start 133.36 47.615) (end 133.36 43.18) (width 0.25) (layer "B.Cu") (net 7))
 (segment (start 64.71 49.575) (end 75.545 49.575) (width 0.25) (layer "B.Cu") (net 7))
 (segment (start 114.3 48.26) (end 116.205 48.26) (width 0.25) (layer "B.Cu") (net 7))
 (segment (start 63.485 50.8) (end 64.71 49.575) (width 0.25) (layer "B.Cu") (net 7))
 (segment (start 75.545 49.575) (end 76.77 50.8) (width 0.25) (layer "B.Cu") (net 7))
 (segment (start 96.52 74.575) (end 101.6 74.575) (width 0.25) (layer "B.Cu") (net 7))
 (segment (start 116.205 73.66) (end 116.205 61.672621) (width 0.25) (layer "B.Cu") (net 7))
 (segment (start 88.89 50.8) (end 90.115 52.025) (width 0.25) (layer "B.Cu") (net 7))
 (segment (start 111.76 74.575) (end 106.68 74.575) (width 0.25) (layer "B.Cu") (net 7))
 (segment (start 116.205 54.522379) (end 116.205 48.26) (width 0.25) (layer "B.Cu") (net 7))
 (segment (start 101.085 52.025) (end 102.87 50.24) (width 0.25) (layer "B.Cu") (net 7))
 (segment (start 87.665 49.575) (end 77.995 49.575) (width 0.25) (layer "B.Cu") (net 7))
 (segment (start 105.7025 43.18) (end 102.87 46.0125) (width 0.25) (layer "B.Cu") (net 7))
 (segment (start 101.6 74.575) (end 106.68 74.575) (width 0.25) (layer "B.Cu") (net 7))
 (segment (start 115.29 74.575) (end 116.205 73.66) (width 0.25) (layer "B.Cu") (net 7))
 (segment (start 116.205 48.26) (end 132.715 48.26) (width 0.25) (layer "B.Cu") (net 7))
 (segment (start 132.715 48.26) (end 133.36 47.615) (width 0.25) (layer "B.Cu") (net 7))
 (segment (start 86.36 55.88) (end 86.35 55.87) (width 0.25) (layer "B.Cu") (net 11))
 (segment (start 86.35 55.87) (end 86.35 50.8) (width 0.25) (layer "B.Cu") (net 11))
 (segment (start 91.43 45.99) (end 91.43 50.8) (width 0.25) (layer "B.Cu") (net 12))
 (segment (start 91.16 45.72) (end 91.43 45.99) (width 0.25) (layer "B.Cu") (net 12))
 (segment (start 74.015 55.88) (end 74.23 55.665) (width 0.25) (layer "B.Cu") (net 6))
 (segment (start 74.23 55.665) (end 74.23 50.8) (width 0.25) (layer "B.Cu") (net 6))
 (segment (start 60.96 55.88) (end 60.945 55.865) (width 0.25) (layer "B.Cu") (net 13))
 (segment (start 60.945 55.865) (end 60.945 50.8) (width 0.25) (layer "B.Cu") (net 13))
 (segment (start 109.23 53.34) (end 121.285 53.34) (width 0.25) (layer "F.Cu") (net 21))
 (segment (start 106.69 50.8) (end 109.23 53.34) (width 0.25) (layer "F.Cu") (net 21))
 (via (at 121.285 53.34) (size 0.8) (drill 0.4) (layers "F.Cu" "B.Cu") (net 21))
 (segment (start 155.575 58.42) (end 160.02 58.42) (width 0.25) (layer "B.Cu") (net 21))
 (segment (start 121.285 53.34) (end 150.495 53.34) (width 0.25) (layer "B.Cu") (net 21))
 (segment (start 150.495 53.34) (end 155.575 58.42) (width 0.25) (layer "B.Cu") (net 21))
 (segment (start 102.87 53.34) (end 105.41 50.8) (width 0.25) (layer "B.Cu") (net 21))
 (segment (start 105.41 50.8) (end 106.69 50.8) (width 0.25) (layer "B.Cu") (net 21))
 (segment (start 96.52 71.475) (end 96.52 67.945) (width 0.25) (layer "B.Cu") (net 22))
 (segment (start 101.6 67.945) (end 106.69 62.855) (width 0.25) (layer "B.Cu") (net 19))
 (segment (start 101.6 71.475) (end 101.6 67.945) (width 0.25) (layer "B.Cu") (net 19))
 (segment (start 106.69 62.855) (end 106.69 60.96) (width 0.25) (layer "B.Cu") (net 19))
 (segment (start 106.68 67.945) (end 106.68 71.475) (width 0.25) (layer "B.Cu") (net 23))
 (segment (start 106.69 58.42) (end 111.76 63.49) (width 0.25) (layer "B.Cu") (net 20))
 (segment (start 111.76 63.49) (end 111.76 67.945) (width 0.25) (layer "B.Cu") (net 20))
 (segment (start 111.76 71.475) (end 111.76 67.945) (width 0.25) (layer "B.Cu") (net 20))
 (segment (start 163.195 58.42) (end 163.195 69.85) (width 0.25) (layer "B.Cu") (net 8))
 (segment (start 168.2 70.195) (end 174.7 70.195) (width 0.25) (layer "B.Cu") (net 8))
 (segment (start 163.54 70.195) (end 168.2 70.195) (width 0.25) (layer "B.Cu") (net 8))
 (segment (start 163.195 69.85) (end 163.54 70.195) (width 0.25) (layer "B.Cu") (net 8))
 (segment (start 160.02 55.875) (end 160.65 55.875) (width 0.25) (layer "B.Cu") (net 8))
 (segment (start 160.65 55.875) (end 163.195 58.42) (width 0.25) (layer "B.Cu") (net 8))
 (segment (start 179.705 55.245) (end 180.34 54.61) (width 0.25) (layer "B.Cu") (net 5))
 (segment (start 180.34 54.61) (end 180.34 48.895) (width 0.25) (layer "B.Cu") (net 5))
 (segment (start 179.745 48.3) (end 178.58 48.3) (width 0.25) (layer "B.Cu") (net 5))
 (segment (start 161.93 55.245) (end 179.705 55.245) (width 0.25) (layer "B.Cu") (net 5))
 (segment (start 160.02 53.335) (end 161.93 55.245) (width 0.25) (layer "B.Cu") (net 5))
 (segment (start 180.34 48.895) (end 179.745 48.3) (width 0.25) (layer "B.Cu") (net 5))
 (segment (start 160.02 50.795) (end 161.575 50.795) (width 0.25) (layer "B.Cu") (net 4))
 (segment (start 161.575 50.795) (end 164.08 53.3) (width 0.25) (layer "B.Cu") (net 4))
 (segment (start 164.035 48.255) (end 164.08 48.3) (width 0.25) (layer "B.Cu") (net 3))
 (segment (start 160.02 48.255) (end 164.035 48.255) (width 0.25) (layer "B.Cu") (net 3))
 (segment (start 107.95 48.26) (end 110.49 45.72) (width 0.25) (layer "B.Cu") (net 9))
 (segment (start 138.44 43.18) (end 137.265 42.005) (width 0.25) (layer "B.Cu") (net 9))
 (segment (start 106.69 48.26) (end 107.95 48.26) (width 0.25) (layer "B.Cu") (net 9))
 (segment (start 110.49 45.72) (end 114.3 45.72) (width 0.25) (layer "B.Cu") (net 9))
 (segment (start 118.015 42.005) (end 114.3 45.72) (width 0.25) (layer "B.Cu") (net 9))
 (segment (start 137.265 42.005) (end 118.015 42.005) (width 0.25) (layer "B.Cu") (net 9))
 (segment (start 110.49 43.18) (end 114.3 43.18) (width 0.25) (layer "B.Cu") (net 10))
 (segment (start 116.205 41.275) (end 140.335 41.275) (width 0.25) (layer "B.Cu") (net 10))
 (segment (start 114.3 43.18) (end 116.205 41.275) (width 0.25) (layer "B.Cu") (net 10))
 (segment (start 140.335 41.275) (end 140.98 41.92) (width 0.25) (layer "B.Cu") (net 10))
 (segment (start 140.98 41.92) (end 140.98 43.18) (width 0.25) (layer "B.Cu") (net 10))
 (segment (start 107.95 45.72) (end 110.49 43.18) (width 0.25) (layer "B.Cu") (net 10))
 (segment (start 106.69 45.72) (end 107.95 45.72) (width 0.25) (layer "B.Cu") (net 10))
 (segment (start 104.14 63.5) (end 104.14 58.97901) (width 0.25) (layer "B.Cu") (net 2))
 (segment (start 108.215 56.34599) (end 108.215 54.865) (width 0.25) (layer "B.Cu") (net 2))
 (segment (start 104.14 58.97901) (end 106.11401 57.005) (width 0.25) (layer "B.Cu") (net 2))
 (segment (start 103.505 64.135) (end 104.14 63.5) (width 0.25) (layer "B.Cu") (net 2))
 (segment (start 72.24 65.695) (end 78.74 65.695) (width 0.25) (layer "B.Cu") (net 2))
 (segment (start 107.55599 57.005) (end 108.215 56.34599) (width 0.25) (layer "B.Cu") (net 2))
 (segment (start 93 67.02) (end 95.885 64.135) (width 0.25) (layer "B.Cu") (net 2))
 (segment (start 80.065 67.02) (end 93 67.02) (width 0.25) (layer "B.Cu") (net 2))
 (segment (start 78.74 65.695) (end 80.065 67.02) (width 0.25) (layer "B.Cu") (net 2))
 (segment (start 95.885 64.135) (end 103.505 64.135) (width 0.25) (layer "B.Cu") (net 2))
 (segment (start 106.11401 57.005) (end 107.55599 57.005) (width 0.25) (layer "B.Cu") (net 2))
 (segment (start 108.215 54.865) (end 106.69 53.34) (width 0.25) (layer "B.Cu") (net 2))
 (segment (start 92.15 65.695) (end 94.98 62.865) (width 0.25) (layer "B.Cu") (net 14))
 (segment (start 103.505 55.88) (end 106.69 55.88) (width 0.25) (layer "B.Cu") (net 14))
 (segment (start 102.87 62.23) (end 102.87 56.515) (width 0.25) (layer "B.Cu") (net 14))
 (segment (start 94.98 62.865) (end 102.235 62.865) (width 0.25) (layer "B.Cu") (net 14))
 (segment (start 102.87 56.515) (end 103.505 55.88) (width 0.25) (layer "B.Cu") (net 14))
 (segment (start 85.65 65.695) (end 92.15 65.695) (width 0.25) (layer "B.Cu") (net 14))
 (segment (start 102.235 62.865) (end 102.87 62.23) (width 0.25) (layer "B.Cu") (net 14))
 (segment (start 97.155 55.88) (end 99.07 55.88) (width 0.25) (layer "B.Cu") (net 17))
 (segment (start 95.25 57.785) (end 97.155 55.88) (width 0.25) (layer "B.Cu") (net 17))
 (segment (start 77.115 55.88) (end 82.55 55.88) (width 0.25) (layer "B.Cu") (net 17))
 (segment (start 82.55 55.88) (end 84.455 57.785) (width 0.25) (layer "B.Cu") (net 17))
 (segment (start 84.455 57.785) (end 95.25 57.785) (width 0.25) (layer "B.Cu") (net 17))
 (segment (start 64.06 57.075) (end 64.06 55.88) (width 0.25) (layer "B.Cu") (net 18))
 (segment (start 65.405 58.42) (end 64.06 57.075) (width 0.25) (layer "B.Cu") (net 18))
 (segment (start 99.07 58.42) (end 65.405 58.42) (width 0.25) (layer "B.Cu") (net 18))
 (segment (start 94.26 48.54) (end 94.26 45.72) (width 0.25) (layer "B.Cu") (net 15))
 (segment (start 96.52 50.8) (end 94.26 48.54) (width 0.25) (layer "B.Cu") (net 15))
 (segment (start 99.07 50.8) (end 96.52 50.8) (width 0.25) (layer "B.Cu") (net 15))
 (segment (start 99.07 53.34) (end 90.805 53.34) (width 0.25) (layer "B.Cu") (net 16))
 (segment (start 90.805 53.34) (end 89.46 54.685) (width 0.25) (layer "B.Cu") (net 16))
 (segment (start 89.46 54.685) (end 89.46 55.88) (width 0.25) (layer "B.Cu") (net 16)))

